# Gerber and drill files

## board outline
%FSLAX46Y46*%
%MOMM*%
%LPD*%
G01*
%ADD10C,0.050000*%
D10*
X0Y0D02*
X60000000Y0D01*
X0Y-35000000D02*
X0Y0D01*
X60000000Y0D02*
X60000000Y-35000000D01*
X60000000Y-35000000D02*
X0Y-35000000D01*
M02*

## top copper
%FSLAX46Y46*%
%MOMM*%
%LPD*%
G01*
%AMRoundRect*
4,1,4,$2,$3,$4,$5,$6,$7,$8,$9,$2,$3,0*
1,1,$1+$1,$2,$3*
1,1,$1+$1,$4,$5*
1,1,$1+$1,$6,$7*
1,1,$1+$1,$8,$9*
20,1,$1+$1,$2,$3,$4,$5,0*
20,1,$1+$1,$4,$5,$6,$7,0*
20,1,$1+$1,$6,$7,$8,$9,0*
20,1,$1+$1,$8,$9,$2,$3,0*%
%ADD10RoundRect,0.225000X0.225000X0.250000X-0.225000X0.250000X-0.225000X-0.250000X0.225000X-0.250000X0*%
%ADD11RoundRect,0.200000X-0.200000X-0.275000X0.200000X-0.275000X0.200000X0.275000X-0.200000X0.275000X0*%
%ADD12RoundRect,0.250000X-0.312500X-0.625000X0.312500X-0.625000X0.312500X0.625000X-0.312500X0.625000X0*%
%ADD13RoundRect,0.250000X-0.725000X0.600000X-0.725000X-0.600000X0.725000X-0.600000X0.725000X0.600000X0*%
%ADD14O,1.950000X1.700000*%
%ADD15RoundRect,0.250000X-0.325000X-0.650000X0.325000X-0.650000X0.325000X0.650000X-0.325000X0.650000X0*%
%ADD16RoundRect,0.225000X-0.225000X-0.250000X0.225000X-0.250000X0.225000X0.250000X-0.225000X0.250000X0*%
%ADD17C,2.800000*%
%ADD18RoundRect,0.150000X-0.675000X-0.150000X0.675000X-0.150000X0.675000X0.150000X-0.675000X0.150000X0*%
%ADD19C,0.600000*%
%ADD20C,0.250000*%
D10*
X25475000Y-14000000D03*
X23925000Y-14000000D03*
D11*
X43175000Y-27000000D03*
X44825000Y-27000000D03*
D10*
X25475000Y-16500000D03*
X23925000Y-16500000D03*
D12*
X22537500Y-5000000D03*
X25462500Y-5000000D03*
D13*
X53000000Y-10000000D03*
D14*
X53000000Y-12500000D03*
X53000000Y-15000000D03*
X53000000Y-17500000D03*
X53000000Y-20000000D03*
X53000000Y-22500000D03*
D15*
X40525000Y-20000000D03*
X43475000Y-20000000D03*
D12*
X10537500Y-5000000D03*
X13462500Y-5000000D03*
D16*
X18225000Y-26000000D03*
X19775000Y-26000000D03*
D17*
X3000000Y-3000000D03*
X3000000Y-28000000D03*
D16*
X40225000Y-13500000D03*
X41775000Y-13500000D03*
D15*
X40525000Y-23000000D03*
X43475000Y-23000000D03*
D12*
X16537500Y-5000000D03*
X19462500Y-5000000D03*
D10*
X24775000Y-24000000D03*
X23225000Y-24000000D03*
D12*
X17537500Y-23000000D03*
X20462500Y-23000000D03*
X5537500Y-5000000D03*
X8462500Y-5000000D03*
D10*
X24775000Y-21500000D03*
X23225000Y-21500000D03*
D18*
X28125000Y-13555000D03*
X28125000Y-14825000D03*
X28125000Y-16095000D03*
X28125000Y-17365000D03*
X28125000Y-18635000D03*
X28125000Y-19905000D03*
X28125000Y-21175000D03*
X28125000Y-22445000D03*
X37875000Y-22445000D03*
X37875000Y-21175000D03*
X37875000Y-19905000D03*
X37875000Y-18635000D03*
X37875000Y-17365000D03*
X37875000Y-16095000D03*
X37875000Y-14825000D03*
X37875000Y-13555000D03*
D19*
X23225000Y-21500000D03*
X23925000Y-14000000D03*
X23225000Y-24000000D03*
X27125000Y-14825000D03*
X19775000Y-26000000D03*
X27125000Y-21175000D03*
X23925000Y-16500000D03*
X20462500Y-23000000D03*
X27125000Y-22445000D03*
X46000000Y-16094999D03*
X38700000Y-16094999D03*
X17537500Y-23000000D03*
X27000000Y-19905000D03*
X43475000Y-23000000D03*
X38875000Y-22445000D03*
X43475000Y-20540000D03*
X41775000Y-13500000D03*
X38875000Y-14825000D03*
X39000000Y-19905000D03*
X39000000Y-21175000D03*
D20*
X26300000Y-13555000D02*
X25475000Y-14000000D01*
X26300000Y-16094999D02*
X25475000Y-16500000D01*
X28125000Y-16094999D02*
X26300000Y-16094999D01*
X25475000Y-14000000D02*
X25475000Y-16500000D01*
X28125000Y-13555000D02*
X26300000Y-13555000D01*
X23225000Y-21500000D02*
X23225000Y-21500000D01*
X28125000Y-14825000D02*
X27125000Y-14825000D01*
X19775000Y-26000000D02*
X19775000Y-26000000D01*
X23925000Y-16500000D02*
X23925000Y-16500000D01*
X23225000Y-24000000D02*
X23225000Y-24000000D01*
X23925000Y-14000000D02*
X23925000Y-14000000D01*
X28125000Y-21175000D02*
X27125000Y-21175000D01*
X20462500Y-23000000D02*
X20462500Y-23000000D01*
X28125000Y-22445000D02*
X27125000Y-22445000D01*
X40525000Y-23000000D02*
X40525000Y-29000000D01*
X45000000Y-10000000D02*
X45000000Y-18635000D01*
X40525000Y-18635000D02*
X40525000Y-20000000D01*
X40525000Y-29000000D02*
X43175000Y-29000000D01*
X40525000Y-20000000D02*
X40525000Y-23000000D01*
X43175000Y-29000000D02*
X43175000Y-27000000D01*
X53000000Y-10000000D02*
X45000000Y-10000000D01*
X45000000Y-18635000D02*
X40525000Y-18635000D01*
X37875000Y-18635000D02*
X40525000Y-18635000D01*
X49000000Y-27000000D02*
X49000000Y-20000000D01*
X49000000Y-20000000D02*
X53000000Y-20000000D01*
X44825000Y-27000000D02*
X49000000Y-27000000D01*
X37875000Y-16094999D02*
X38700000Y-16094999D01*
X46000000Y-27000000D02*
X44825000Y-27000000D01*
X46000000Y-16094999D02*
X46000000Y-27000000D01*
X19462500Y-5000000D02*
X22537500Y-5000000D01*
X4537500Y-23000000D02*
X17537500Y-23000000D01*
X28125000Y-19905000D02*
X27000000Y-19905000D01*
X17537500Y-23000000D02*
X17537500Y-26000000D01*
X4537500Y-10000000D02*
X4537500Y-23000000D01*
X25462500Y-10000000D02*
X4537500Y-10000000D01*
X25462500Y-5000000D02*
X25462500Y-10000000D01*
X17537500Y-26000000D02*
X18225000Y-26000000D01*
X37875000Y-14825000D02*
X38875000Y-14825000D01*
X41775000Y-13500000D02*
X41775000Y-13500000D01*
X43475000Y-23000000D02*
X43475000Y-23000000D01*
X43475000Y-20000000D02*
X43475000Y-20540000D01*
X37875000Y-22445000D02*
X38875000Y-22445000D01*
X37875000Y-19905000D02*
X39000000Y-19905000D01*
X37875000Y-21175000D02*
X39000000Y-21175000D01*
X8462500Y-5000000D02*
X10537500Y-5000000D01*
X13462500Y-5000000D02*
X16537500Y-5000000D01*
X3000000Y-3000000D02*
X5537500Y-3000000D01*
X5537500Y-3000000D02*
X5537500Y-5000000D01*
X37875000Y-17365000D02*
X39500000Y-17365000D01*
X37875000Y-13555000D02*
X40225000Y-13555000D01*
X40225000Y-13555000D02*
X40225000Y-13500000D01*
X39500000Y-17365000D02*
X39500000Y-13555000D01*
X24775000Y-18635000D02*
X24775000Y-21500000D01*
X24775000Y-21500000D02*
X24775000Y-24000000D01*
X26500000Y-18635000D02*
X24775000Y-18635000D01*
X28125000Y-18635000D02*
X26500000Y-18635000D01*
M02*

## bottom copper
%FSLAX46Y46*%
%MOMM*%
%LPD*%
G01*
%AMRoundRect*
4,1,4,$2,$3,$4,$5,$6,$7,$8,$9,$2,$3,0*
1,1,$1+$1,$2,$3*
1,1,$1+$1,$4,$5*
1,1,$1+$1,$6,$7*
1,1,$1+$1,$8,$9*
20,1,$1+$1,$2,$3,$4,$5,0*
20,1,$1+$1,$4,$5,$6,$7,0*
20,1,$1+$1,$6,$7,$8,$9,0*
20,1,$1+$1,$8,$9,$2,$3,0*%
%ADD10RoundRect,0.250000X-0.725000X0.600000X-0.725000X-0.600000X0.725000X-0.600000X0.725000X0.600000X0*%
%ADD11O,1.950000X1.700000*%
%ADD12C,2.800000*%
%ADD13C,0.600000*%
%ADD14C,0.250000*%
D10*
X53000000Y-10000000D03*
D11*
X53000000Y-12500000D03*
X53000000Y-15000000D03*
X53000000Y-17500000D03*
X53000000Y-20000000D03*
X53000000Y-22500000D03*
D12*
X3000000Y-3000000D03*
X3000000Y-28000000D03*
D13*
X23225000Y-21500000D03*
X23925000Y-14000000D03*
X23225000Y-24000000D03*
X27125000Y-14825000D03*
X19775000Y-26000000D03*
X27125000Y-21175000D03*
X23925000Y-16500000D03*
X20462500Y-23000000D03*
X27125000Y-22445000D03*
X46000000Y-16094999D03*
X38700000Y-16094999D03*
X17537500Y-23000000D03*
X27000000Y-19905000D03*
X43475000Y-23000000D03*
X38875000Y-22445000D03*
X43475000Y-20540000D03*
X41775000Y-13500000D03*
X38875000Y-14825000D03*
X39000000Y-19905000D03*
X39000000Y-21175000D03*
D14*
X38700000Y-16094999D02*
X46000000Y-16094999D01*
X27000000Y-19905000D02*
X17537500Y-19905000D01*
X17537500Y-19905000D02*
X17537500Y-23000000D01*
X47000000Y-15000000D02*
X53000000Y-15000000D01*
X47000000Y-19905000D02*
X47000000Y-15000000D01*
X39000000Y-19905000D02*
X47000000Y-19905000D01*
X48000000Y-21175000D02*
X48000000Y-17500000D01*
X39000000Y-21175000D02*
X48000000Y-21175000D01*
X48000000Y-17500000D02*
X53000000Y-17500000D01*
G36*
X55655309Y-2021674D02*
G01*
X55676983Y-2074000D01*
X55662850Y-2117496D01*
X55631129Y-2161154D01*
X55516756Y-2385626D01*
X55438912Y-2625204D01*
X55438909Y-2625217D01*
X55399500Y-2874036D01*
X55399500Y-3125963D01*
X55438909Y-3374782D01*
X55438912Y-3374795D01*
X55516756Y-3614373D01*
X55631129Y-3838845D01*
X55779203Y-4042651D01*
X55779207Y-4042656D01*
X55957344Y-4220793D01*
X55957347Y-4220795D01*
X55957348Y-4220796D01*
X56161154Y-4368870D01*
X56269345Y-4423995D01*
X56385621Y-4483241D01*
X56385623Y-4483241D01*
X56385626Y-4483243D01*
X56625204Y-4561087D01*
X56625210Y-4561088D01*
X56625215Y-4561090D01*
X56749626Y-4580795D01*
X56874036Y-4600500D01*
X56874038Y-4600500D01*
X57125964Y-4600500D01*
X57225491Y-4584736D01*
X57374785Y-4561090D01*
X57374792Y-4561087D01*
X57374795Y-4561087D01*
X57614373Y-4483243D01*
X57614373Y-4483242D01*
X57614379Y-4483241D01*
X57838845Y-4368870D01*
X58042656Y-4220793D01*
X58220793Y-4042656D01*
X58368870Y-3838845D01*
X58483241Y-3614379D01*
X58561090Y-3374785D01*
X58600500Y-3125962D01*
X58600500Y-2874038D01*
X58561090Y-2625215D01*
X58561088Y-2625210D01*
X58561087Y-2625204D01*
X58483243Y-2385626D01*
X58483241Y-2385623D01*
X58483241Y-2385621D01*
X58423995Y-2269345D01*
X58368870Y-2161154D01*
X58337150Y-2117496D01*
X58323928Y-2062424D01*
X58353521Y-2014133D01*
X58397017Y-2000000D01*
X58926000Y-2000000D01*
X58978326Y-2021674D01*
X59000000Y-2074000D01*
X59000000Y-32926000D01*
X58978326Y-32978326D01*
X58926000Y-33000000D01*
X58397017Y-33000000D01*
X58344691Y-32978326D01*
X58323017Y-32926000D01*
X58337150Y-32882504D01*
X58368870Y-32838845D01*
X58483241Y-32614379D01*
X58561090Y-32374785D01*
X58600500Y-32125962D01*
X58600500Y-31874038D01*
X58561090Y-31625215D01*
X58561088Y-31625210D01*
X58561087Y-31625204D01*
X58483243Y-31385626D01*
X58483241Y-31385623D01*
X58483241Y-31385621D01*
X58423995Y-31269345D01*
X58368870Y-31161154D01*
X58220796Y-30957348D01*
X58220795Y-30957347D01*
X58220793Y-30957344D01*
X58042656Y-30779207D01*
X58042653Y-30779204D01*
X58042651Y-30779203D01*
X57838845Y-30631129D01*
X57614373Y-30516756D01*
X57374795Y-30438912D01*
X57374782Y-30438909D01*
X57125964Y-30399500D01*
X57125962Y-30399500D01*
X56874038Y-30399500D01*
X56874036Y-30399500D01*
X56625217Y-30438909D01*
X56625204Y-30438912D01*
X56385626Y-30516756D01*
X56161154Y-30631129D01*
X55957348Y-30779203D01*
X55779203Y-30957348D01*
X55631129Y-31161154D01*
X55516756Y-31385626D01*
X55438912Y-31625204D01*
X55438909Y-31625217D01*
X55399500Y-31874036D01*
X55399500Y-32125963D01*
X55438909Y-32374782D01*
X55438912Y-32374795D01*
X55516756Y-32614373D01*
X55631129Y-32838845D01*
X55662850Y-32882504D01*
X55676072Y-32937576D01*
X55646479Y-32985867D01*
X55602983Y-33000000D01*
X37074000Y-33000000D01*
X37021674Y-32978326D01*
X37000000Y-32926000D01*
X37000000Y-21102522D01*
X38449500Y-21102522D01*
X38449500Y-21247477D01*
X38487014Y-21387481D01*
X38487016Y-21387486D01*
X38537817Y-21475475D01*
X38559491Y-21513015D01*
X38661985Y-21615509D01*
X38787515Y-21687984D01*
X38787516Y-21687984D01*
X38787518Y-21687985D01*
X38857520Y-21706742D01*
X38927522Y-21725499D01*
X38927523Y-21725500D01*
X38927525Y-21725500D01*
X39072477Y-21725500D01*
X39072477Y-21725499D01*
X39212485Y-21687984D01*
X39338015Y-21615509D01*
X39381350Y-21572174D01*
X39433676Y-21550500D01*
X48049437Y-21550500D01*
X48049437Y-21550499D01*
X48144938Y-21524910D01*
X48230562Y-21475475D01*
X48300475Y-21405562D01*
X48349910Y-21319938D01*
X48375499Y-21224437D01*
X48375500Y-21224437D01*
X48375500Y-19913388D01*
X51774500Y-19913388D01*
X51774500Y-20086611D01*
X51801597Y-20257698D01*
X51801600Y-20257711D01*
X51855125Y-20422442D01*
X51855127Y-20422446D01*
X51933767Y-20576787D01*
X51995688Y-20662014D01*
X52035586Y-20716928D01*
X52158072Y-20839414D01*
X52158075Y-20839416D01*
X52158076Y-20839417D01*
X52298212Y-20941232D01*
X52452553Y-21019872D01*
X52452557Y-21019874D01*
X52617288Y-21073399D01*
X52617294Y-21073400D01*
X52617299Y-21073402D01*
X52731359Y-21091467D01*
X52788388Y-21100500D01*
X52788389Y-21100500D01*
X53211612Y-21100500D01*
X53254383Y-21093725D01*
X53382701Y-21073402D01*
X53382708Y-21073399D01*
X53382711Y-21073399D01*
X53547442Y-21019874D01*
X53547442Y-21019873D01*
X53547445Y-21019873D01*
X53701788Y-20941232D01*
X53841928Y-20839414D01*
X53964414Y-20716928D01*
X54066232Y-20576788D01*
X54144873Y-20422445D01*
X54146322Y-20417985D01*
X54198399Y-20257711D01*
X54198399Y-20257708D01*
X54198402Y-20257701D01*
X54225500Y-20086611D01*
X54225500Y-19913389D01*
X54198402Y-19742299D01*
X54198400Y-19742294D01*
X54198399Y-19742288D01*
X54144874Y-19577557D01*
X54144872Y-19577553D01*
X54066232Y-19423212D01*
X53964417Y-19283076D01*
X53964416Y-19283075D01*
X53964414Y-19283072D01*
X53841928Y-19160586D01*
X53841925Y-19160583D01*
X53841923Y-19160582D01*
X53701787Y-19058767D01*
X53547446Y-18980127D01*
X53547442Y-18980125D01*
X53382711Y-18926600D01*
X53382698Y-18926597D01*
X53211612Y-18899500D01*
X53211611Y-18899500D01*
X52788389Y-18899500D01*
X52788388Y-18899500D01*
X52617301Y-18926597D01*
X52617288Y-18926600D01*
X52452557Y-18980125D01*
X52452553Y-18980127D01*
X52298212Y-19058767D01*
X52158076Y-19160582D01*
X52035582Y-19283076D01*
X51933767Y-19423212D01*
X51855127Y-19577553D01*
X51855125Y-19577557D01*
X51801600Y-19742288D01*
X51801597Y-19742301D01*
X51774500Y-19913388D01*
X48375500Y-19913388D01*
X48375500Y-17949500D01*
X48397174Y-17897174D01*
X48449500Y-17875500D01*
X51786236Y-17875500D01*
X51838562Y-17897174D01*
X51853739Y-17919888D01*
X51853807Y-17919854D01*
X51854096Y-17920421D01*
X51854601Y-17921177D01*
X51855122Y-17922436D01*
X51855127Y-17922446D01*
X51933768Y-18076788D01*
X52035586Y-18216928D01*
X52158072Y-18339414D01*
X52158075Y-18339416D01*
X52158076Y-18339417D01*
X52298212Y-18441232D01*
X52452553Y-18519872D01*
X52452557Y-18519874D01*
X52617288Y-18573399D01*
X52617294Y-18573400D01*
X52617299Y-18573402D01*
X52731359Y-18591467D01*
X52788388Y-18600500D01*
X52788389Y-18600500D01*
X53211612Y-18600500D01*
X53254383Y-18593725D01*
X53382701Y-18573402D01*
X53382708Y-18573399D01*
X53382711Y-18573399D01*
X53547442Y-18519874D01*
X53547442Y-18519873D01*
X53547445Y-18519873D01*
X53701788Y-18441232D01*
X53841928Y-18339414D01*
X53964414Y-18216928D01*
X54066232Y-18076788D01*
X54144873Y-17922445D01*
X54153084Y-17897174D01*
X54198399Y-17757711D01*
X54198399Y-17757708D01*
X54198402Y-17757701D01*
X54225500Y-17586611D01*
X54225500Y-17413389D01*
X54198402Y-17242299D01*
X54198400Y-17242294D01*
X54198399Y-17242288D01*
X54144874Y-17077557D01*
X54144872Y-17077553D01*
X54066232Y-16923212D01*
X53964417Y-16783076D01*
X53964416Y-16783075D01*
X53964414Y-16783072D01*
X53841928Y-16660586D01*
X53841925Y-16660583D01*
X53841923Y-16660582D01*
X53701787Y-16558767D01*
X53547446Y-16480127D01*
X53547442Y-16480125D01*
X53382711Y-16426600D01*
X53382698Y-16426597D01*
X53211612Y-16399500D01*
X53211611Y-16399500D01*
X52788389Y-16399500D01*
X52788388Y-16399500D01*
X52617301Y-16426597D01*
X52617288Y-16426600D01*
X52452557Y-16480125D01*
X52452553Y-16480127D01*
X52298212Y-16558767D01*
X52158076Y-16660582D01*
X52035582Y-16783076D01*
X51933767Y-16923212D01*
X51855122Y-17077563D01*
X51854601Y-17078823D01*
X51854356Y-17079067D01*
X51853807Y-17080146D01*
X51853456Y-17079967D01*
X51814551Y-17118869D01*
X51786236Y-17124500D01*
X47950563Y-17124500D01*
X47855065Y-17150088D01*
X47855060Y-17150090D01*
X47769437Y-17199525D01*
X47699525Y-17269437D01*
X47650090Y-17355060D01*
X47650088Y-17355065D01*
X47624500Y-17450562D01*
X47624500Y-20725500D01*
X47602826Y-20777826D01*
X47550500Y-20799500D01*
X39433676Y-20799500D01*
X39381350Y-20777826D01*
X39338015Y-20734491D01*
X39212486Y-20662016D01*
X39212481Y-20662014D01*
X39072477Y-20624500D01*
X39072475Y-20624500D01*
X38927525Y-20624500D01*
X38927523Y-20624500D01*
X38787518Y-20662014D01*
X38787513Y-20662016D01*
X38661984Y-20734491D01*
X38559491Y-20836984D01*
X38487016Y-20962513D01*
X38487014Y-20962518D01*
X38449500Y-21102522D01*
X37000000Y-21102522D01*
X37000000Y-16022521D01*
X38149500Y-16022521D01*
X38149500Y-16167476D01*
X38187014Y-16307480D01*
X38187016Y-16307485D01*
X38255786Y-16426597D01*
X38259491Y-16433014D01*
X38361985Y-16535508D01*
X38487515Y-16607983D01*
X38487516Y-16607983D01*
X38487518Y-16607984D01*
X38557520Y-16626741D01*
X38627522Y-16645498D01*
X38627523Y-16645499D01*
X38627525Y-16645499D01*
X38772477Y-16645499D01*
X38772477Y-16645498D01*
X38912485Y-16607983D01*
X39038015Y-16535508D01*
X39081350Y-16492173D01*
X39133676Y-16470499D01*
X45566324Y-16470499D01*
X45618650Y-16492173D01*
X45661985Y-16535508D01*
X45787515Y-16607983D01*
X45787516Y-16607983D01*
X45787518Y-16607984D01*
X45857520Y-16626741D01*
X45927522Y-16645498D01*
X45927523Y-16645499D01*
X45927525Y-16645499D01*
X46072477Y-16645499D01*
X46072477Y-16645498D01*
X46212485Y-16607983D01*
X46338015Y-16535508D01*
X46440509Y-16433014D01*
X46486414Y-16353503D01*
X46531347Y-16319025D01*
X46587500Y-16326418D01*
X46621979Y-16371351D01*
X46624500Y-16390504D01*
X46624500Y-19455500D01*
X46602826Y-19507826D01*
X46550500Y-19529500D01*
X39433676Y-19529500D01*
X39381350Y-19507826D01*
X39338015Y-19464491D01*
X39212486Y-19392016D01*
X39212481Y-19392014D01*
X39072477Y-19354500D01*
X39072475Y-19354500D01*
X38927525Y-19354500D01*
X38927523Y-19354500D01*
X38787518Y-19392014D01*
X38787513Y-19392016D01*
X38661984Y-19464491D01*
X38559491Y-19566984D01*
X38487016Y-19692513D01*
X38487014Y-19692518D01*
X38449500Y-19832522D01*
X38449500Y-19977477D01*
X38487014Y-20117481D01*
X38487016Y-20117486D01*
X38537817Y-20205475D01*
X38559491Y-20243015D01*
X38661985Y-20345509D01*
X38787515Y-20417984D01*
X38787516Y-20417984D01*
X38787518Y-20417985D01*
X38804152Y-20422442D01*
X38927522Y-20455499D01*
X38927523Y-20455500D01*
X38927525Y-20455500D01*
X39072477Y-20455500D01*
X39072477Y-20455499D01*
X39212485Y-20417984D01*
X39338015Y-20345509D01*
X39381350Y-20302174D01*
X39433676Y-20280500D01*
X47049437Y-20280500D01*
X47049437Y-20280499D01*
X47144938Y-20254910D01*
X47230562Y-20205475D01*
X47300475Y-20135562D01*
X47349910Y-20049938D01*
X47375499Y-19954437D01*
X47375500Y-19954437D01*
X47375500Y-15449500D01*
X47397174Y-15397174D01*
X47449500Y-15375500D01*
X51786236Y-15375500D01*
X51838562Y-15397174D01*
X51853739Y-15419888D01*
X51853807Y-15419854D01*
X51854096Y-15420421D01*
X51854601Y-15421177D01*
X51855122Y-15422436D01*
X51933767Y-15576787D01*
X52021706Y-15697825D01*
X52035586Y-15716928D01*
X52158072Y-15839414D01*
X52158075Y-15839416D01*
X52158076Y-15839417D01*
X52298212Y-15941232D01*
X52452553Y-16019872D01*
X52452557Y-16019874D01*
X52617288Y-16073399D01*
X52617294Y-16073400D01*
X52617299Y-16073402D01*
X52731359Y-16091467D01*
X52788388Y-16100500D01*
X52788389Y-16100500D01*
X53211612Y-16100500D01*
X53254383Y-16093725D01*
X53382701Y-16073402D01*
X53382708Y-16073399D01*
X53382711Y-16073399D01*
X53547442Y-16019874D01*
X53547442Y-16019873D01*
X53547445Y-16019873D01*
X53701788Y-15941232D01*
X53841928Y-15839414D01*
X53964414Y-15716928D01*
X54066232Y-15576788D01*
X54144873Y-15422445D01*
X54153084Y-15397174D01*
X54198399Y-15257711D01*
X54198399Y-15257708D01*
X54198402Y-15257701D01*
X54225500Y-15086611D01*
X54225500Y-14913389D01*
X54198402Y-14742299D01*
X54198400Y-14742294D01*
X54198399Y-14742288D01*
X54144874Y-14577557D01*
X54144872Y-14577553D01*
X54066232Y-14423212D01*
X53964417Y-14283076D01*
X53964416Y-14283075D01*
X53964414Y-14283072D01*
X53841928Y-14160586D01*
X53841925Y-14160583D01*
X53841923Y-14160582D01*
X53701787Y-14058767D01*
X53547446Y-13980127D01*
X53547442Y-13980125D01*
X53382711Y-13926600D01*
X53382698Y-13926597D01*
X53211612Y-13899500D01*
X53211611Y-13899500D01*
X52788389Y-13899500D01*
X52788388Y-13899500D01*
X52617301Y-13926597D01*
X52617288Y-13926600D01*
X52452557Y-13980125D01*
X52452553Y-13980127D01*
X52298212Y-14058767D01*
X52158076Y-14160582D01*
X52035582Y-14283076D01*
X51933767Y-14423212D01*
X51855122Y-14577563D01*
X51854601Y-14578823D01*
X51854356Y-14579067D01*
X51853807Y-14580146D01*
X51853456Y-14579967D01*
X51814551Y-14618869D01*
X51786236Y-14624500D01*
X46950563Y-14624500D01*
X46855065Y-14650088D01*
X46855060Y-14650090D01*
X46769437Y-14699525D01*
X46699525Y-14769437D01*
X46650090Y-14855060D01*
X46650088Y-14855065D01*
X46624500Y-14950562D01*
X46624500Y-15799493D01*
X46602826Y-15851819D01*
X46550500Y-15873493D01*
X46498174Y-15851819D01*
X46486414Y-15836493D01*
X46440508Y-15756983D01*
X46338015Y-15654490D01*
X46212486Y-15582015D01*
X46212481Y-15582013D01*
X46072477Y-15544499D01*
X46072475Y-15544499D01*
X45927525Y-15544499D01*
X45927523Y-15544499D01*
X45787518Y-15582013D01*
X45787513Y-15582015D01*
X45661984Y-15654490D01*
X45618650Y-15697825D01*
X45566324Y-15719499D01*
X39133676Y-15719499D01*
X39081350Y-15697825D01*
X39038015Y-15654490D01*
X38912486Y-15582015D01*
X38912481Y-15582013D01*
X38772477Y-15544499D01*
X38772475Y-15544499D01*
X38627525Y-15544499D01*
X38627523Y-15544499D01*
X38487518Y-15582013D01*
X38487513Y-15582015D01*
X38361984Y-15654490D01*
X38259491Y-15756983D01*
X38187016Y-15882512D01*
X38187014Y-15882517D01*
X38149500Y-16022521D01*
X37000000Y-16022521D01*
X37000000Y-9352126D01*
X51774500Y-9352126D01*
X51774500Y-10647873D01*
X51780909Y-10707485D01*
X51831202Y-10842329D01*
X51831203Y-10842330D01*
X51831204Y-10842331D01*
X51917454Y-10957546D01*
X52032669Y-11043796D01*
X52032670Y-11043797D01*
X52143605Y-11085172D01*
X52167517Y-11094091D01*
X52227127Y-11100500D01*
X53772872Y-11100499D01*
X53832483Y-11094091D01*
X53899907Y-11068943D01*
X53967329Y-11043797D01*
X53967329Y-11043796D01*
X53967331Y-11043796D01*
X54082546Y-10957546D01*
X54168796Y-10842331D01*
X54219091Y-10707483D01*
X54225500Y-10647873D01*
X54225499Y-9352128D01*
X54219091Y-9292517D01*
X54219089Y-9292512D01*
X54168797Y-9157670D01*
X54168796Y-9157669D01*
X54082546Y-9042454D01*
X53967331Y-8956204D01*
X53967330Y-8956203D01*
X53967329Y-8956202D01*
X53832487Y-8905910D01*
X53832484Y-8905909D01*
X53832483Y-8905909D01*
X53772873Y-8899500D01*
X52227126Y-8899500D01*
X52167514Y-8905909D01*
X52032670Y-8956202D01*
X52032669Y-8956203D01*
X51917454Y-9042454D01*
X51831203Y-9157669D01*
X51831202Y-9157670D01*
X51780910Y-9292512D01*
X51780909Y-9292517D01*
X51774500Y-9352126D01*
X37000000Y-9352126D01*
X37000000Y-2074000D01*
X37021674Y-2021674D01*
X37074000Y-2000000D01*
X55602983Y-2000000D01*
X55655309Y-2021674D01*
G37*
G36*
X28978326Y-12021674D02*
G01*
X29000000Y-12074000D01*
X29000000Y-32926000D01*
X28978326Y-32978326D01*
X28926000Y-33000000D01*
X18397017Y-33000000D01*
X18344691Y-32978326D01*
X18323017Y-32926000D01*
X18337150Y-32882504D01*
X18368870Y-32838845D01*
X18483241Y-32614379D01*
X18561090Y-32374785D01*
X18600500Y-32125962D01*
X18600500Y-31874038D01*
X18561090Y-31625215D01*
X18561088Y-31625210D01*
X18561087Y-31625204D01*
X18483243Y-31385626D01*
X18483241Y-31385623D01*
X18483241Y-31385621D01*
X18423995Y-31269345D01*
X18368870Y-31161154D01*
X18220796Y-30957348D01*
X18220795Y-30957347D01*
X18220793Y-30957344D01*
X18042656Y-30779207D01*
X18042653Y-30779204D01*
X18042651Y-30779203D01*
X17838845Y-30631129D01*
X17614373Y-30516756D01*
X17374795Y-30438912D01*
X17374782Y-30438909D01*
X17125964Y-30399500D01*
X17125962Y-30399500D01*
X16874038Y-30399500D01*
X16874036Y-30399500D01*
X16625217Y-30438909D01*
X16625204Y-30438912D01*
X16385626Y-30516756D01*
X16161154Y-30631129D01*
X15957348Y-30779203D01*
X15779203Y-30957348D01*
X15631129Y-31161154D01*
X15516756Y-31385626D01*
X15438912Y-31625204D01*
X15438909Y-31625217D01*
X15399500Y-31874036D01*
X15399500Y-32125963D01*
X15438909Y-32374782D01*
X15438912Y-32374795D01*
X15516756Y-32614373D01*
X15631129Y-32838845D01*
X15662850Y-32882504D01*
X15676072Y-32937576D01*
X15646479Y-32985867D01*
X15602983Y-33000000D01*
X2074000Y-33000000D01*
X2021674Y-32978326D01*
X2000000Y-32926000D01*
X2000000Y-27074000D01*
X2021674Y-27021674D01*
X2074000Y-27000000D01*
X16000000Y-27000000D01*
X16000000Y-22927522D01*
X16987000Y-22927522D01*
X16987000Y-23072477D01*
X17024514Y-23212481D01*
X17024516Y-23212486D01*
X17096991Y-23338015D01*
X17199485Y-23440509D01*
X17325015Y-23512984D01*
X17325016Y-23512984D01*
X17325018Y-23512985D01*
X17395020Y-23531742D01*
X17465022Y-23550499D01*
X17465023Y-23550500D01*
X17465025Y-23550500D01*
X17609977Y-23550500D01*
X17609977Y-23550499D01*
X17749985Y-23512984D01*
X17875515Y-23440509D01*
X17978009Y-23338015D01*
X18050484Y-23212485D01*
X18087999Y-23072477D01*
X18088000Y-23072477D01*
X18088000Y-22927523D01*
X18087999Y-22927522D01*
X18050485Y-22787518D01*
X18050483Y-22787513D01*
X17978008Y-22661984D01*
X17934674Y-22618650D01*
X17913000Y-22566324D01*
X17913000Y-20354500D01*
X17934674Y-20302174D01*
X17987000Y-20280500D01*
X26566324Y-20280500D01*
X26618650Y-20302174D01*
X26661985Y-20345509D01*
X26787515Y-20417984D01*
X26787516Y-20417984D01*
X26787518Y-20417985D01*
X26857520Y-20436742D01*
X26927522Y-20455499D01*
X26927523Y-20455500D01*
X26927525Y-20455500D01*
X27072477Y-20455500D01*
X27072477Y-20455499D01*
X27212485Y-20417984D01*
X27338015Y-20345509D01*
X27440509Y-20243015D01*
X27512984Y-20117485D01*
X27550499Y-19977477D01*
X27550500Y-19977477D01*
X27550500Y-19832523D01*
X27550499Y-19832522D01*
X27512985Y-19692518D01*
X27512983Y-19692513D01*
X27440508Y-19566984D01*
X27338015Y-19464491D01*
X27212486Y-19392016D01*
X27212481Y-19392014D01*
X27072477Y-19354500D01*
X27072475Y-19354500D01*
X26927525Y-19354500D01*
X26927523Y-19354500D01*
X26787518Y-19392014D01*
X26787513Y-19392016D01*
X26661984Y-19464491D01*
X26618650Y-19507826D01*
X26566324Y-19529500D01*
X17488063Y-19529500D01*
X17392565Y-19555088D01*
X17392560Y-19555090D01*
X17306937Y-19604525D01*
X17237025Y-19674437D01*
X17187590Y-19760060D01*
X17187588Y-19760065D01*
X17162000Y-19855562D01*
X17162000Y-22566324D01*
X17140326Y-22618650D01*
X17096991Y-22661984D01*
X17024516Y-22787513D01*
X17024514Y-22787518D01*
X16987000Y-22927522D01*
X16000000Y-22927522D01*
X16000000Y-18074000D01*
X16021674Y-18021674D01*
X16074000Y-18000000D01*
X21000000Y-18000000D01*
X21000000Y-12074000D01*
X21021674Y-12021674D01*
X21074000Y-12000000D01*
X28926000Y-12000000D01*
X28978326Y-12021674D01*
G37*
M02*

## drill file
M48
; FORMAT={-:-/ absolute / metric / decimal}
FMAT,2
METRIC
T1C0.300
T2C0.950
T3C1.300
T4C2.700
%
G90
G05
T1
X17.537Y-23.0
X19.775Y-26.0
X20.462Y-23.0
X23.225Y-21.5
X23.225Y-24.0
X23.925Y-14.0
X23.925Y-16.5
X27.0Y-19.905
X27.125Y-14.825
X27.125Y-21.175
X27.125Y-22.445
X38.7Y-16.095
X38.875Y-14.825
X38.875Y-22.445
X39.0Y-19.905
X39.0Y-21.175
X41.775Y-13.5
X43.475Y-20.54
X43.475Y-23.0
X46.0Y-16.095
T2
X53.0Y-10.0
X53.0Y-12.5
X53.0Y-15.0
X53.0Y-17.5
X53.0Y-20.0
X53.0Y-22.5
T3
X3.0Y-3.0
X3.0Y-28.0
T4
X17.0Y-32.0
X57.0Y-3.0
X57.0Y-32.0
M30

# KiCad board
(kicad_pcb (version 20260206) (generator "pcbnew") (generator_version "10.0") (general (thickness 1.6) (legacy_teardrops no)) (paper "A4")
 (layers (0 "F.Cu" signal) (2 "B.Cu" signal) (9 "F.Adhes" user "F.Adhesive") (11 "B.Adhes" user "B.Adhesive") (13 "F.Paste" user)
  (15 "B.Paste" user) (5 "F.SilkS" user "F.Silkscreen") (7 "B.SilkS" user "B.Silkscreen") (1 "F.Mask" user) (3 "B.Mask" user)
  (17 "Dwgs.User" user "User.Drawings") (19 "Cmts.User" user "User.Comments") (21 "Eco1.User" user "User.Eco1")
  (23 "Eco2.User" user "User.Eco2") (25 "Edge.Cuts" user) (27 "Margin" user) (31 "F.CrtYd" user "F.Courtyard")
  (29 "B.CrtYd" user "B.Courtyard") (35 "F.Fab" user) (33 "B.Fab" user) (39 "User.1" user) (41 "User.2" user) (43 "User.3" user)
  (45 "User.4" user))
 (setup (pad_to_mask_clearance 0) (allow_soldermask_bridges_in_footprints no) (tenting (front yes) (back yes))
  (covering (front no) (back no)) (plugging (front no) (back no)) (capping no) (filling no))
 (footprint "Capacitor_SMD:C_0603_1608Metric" (layer "F.Cu") (at 24.7 14 180)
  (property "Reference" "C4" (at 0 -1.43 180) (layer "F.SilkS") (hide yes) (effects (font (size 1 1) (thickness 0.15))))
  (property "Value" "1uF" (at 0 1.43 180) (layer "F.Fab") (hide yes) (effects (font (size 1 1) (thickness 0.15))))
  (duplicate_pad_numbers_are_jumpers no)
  (pad "1" smd roundrect (at -0.775 0 180) (size 0.9 0.95) (layers "F.Cu" "F.Mask" "F.Paste") (roundrect_rratio 0.25) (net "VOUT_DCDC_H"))
  (pad "2" smd roundrect (at 0.775 0 180) (size 0.9 0.95) (layers "F.Cu" "F.Mask" "F.Paste") (roundrect_rratio 0.25) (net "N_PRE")))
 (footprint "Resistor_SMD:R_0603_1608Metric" (layer "F.Cu") (at 44 27)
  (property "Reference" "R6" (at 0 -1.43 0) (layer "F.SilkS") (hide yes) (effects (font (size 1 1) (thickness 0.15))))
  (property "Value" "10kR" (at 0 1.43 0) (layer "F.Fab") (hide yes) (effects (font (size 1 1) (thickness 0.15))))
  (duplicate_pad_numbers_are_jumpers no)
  (pad "1" smd roundrect (at -0.825 0) (size 0.8 0.95) (layers "F.Cu" "F.Mask" "F.Paste") (roundrect_rratio 0.25) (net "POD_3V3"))
  (pad "2" smd roundrect (at 0.825 0) (size 0.8 0.95) (layers "F.Cu" "F.Mask" "F.Paste") (roundrect_rratio 0.25) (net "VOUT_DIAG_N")))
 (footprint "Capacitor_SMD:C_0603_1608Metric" (layer "F.Cu") (at 24.7 16.5 180)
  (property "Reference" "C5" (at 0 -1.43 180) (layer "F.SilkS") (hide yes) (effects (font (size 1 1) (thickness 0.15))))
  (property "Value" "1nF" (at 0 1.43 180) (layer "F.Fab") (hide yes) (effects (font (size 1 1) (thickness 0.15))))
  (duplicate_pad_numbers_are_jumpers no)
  (pad "1" smd roundrect (at -0.775 0 180) (size 0.9 0.95) (layers "F.Cu" "F.Mask" "F.Paste") (roundrect_rratio 0.25) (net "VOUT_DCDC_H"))
  (pad "2" smd roundrect (at 0.775 0 180) (size 0.9 0.95) (layers "F.Cu" "F.Mask" "F.Paste") (roundrect_rratio 0.25) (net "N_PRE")))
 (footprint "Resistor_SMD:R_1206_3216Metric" (layer "F.Cu") (at 24 5)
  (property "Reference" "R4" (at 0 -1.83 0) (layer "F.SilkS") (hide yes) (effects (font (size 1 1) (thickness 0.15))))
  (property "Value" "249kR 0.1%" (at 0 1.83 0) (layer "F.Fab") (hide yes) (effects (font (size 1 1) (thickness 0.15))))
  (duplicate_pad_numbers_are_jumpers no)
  (pad "1" smd roundrect (at -1.4625 0) (size 1.125 1.75) (layers "F.Cu" "F.Mask" "F.Paste") (roundrect_rratio 0.222222) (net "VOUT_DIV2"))
  (pad "2" smd roundrect (at 1.4625 0) (size 1.125 1.75) (layers "F.Cu" "F.Mask" "F.Paste") (roundrect_rratio 0.222222) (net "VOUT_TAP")))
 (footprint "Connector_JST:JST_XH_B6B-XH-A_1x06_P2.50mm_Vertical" (layer "F.Cu") (at 53 10 -90)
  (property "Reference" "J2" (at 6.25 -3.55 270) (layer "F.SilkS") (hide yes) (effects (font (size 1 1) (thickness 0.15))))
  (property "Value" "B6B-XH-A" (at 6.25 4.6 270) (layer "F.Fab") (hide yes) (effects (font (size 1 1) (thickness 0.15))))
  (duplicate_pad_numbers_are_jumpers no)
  (pad "1" thru_hole roundrect (at 0 0 270) (size 1.7 1.95) (drill 0.95) (layers "*.Cu" "*.Mask") (remove_unused_layers no)
   (roundrect_rratio 0.147059) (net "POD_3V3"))
  (pad "2" thru_hole oval (at 2.5 0 270) (size 1.7 1.95) (drill 0.95) (layers "*.Cu" "*.Mask") (remove_unused_layers no) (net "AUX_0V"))
  (pad "3" thru_hole oval (at 5 0 270) (size 1.7 1.95) (drill 0.95) (layers "*.Cu" "*.Mask") (remove_unused_layers no) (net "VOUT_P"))
  (pad "4" thru_hole oval (at 7.5 0 270) (size 1.7 1.95) (drill 0.95) (layers "*.Cu" "*.Mask") (remove_unused_layers no) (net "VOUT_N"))
  (pad "5" thru_hole oval (at 10 0 270) (size 1.7 1.95) (drill 0.95) (layers "*.Cu" "*.Mask") (remove_unused_layers no) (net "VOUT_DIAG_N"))
  (pad "6" thru_hole oval (at 12.5 0 270) (size 1.7 1.95) (drill 0.95) (layers "*.Cu" "*.Mask") (remove_unused_layers no) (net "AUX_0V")))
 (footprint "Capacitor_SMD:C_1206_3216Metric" (layer "F.Cu") (at 42 20)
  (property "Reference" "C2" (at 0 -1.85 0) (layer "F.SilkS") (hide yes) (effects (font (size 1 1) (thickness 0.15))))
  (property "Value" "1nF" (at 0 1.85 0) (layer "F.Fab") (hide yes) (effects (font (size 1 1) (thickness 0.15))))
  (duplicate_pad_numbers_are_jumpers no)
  (pad "1" smd roundrect (at -1.475 0) (size 1.15 1.8) (layers "F.Cu" "F.Mask" "F.Paste") (roundrect_rratio 0.217391) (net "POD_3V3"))
  (pad "2" smd roundrect (at 1.475 0) (size 1.15 1.8) (layers "F.Cu" "F.Mask" "F.Paste") (roundrect_rratio 0.217391) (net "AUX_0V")))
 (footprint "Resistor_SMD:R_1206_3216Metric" (layer "F.Cu") (at 12 5)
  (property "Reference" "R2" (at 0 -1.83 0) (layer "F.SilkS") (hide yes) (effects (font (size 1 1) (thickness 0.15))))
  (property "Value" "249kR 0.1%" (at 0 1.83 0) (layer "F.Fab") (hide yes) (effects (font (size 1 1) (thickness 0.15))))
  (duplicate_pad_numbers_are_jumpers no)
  (pad "1" smd roundrect (at -1.4625 0) (size 1.125 1.75) (layers "F.Cu" "F.Mask" "F.Paste") (roundrect_rratio 0.222222) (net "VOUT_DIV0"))
  (pad "2" smd roundrect (at 1.4625 0) (size 1.125 1.75) (layers "F.Cu" "F.Mask" "F.Paste") (roundrect_rratio 0.222222) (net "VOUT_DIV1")))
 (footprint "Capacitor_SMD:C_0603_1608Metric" (layer "F.Cu") (at 19 26)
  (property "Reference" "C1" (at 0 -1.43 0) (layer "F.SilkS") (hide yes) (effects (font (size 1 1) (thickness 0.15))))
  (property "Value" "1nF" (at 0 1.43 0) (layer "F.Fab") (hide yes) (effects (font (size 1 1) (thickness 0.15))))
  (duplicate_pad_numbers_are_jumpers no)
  (pad "1" smd roundrect (at -0.775 0) (size 0.9 0.95) (layers "F.Cu" "F.Mask" "F.Paste") (roundrect_rratio 0.25) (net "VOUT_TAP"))
  (pad "2" smd roundrect (at 0.775 0) (size 0.9 0.95) (layers "F.Cu" "F.Mask" "F.Paste") (roundrect_rratio 0.25) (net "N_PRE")))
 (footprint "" (layer "F.Cu") (at 57 32)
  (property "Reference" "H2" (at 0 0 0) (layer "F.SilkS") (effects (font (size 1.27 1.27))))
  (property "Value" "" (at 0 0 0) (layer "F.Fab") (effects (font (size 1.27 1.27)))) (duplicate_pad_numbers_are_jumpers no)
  (pad "" np_thru_hole circle (at 0 0) (size 2.7 2.7) (drill 2.7) (layers "*.Cu")))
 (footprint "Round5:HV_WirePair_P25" (layer "F.Cu") (at 3 3)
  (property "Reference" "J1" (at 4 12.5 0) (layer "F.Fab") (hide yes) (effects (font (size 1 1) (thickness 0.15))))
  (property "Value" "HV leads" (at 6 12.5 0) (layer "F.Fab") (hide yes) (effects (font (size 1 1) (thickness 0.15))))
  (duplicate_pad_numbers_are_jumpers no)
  (pad "1" thru_hole circle (at 0 0) (size 2.8 2.8) (drill 1.3) (layers "*.Cu" "*.Mask") (remove_unused_layers no) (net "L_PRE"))
  (pad "2" thru_hole circle (at 0 25) (size 2.8 2.8) (drill 1.3) (layers "*.Cu" "*.Mask") (remove_unused_layers no) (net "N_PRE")))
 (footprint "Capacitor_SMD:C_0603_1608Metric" (layer "F.Cu") (at 41 13.5)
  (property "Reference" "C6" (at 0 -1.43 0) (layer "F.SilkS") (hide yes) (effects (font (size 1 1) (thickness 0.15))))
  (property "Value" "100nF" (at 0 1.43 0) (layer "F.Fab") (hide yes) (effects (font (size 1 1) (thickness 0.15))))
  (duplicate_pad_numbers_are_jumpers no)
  (pad "1" smd roundrect (at -0.775 0) (size 0.9 0.95) (layers "F.Cu" "F.Mask" "F.Paste") (roundrect_rratio 0.25) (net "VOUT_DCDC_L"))
  (pad "2" smd roundrect (at 0.775 0) (size 0.9 0.95) (layers "F.Cu" "F.Mask" "F.Paste") (roundrect_rratio 0.25) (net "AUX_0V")))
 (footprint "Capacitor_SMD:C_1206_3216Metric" (layer "F.Cu") (at 42 23)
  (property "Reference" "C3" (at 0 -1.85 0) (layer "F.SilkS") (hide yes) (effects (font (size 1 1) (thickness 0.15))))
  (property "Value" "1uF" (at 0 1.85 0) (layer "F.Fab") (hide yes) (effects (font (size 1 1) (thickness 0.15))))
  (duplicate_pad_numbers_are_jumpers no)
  (pad "1" smd roundrect (at -1.475 0) (size 1.15 1.8) (layers "F.Cu" "F.Mask" "F.Paste") (roundrect_rratio 0.217391) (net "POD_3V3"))
  (pad "2" smd roundrect (at 1.475 0) (size 1.15 1.8) (layers "F.Cu" "F.Mask" "F.Paste") (roundrect_rratio 0.217391) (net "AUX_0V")))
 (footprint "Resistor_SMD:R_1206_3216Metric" (layer "F.Cu") (at 18 5)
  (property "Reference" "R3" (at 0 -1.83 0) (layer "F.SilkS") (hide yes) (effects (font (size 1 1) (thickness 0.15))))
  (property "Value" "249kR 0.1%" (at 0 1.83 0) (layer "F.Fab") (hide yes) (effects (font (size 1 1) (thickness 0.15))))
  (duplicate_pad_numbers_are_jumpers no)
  (pad "1" smd roundrect (at -1.4625 0) (size 1.125 1.75) (layers "F.Cu" "F.Mask" "F.Paste") (roundrect_rratio 0.222222) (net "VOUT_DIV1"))
  (pad "2" smd roundrect (at 1.4625 0) (size 1.125 1.75) (layers "F.Cu" "F.Mask" "F.Paste") (roundrect_rratio 0.222222) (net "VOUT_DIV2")))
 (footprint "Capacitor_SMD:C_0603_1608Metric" (layer "F.Cu") (at 24 24 180)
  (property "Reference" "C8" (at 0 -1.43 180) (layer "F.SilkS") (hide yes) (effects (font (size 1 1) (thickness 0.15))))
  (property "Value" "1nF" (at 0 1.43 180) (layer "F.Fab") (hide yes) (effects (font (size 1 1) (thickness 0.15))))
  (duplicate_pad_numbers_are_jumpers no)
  (pad "1" smd roundrect (at -0.775 0 180) (size 0.9 0.95) (layers "F.Cu" "F.Mask" "F.Paste") (roundrect_rratio 0.25) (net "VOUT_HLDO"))
  (pad "2" smd roundrect (at 0.775 0 180) (size 0.9 0.95) (layers "F.Cu" "F.Mask" "F.Paste") (roundrect_rratio 0.25) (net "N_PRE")))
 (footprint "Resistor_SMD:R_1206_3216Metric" (layer "F.Cu") (at 19 23)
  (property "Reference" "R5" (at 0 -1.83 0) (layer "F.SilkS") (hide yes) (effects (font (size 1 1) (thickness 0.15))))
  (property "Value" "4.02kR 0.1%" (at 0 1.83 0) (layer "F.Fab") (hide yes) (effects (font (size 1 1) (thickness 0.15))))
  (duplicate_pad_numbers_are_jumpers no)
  (pad "1" smd roundrect (at -1.4625 0) (size 1.125 1.75) (layers "F.Cu" "F.Mask" "F.Paste") (roundrect_rratio 0.222222) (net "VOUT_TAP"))
  (pad "2" smd roundrect (at 1.4625 0) (size 1.125 1.75) (layers "F.Cu" "F.Mask" "F.Paste") (roundrect_rratio 0.222222) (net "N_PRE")))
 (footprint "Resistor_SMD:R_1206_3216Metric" (layer "F.Cu") (at 7 5)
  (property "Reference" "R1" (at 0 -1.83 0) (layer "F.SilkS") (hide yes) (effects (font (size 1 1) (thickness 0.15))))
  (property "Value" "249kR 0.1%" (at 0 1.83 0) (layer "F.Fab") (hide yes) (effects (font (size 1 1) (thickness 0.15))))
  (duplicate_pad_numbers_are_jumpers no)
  (pad "1" smd roundrect (at -1.4625 0) (size 1.125 1.75) (layers "F.Cu" "F.Mask" "F.Paste") (roundrect_rratio 0.222222) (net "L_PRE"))
  (pad "2" smd roundrect (at 1.4625 0) (size 1.125 1.75) (layers "F.Cu" "F.Mask" "F.Paste") (roundrect_rratio 0.222222) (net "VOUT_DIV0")))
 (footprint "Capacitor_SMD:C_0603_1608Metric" (layer "F.Cu") (at 24 21.5 180)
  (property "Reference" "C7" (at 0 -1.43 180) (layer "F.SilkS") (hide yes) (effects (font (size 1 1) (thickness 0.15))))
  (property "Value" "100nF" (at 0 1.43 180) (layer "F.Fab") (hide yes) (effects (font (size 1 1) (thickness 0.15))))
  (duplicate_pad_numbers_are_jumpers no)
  (pad "1" smd roundrect (at -0.775 0 180) (size 0.9 0.95) (layers "F.Cu" "F.Mask" "F.Paste") (roundrect_rratio 0.25) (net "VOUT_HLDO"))
  (pad "2" smd roundrect (at 0.775 0 180) (size 0.9 0.95) (layers "F.Cu" "F.Mask" "F.Paste") (roundrect_rratio 0.25) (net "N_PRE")))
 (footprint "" (layer "F.Cu") (at 57 3)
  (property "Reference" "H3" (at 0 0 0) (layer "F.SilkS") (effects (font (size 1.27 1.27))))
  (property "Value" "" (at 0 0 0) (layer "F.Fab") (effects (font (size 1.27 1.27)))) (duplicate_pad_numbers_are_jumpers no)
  (pad "" np_thru_hole circle (at 0 0) (size 2.7 2.7) (drill 2.7) (layers "*.Cu")))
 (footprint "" (layer "F.Cu") (at 17 32)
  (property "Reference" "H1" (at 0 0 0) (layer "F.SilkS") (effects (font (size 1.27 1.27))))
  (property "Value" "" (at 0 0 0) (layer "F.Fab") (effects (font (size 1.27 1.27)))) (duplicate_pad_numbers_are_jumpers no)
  (pad "" np_thru_hole circle (at 0 0) (size 2.7 2.7) (drill 2.7) (layers "*.Cu")))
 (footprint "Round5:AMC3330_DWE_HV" (layer "F.Cu") (at 33 18)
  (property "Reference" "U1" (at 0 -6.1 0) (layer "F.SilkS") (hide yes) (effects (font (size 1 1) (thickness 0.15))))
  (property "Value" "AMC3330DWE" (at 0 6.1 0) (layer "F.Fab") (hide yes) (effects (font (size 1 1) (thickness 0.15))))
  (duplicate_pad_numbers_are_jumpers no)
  (pad "1" smd roundrect (at -4.875 -4.445) (size 1.65 0.6) (layers "F.Cu" "F.Mask" "F.Paste") (roundrect_rratio 0.25) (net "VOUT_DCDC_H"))
  (pad "2" smd roundrect (at -4.875 -3.175) (size 1.65 0.6) (layers "F.Cu" "F.Mask" "F.Paste") (roundrect_rratio 0.25) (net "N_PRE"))
  (pad "3" smd roundrect (at -4.875 -1.905) (size 1.65 0.6) (layers "F.Cu" "F.Mask" "F.Paste") (roundrect_rratio 0.25) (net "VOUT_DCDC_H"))
  (pad "4" smd roundrect (at -4.875 -0.635) (size 1.65 0.6) (layers "F.Cu" "F.Mask" "F.Paste") (roundrect_rratio 0.25)
   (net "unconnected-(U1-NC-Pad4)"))
  (pad "5" smd roundrect (at -4.875 0.635) (size 1.65 0.6) (layers "F.Cu" "F.Mask" "F.Paste") (roundrect_rratio 0.25) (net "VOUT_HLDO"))
  (pad "6" smd roundrect (at -4.875 1.905) (size 1.65 0.6) (layers "F.Cu" "F.Mask" "F.Paste") (roundrect_rratio 0.25) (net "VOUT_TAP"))
  (pad "7" smd roundrect (at -4.875 3.175) (size 1.65 0.6) (layers "F.Cu" "F.Mask" "F.Paste") (roundrect_rratio 0.25) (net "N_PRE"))
  (pad "8" smd roundrect (at -4.875 4.445) (size 1.65 0.6) (layers "F.Cu" "F.Mask" "F.Paste") (roundrect_rratio 0.25) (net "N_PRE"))
  (pad "9" smd roundrect (at 4.875 4.445) (size 1.65 0.6) (layers "F.Cu" "F.Mask" "F.Paste") (roundrect_rratio 0.25) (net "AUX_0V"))
  (pad "10" smd roundrect (at 4.875 3.175) (size 1.65 0.6) (layers "F.Cu" "F.Mask" "F.Paste") (roundrect_rratio 0.25) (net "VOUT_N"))
  (pad "11" smd roundrect (at 4.875 1.905) (size 1.65 0.6) (layers "F.Cu" "F.Mask" "F.Paste") (roundrect_rratio 0.25) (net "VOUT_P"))
  (pad "12" smd roundrect (at 4.875 0.635) (size 1.65 0.6) (layers "F.Cu" "F.Mask" "F.Paste") (roundrect_rratio 0.25) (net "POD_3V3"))
  (pad "13" smd roundrect (at 4.875 -0.635) (size 1.65 0.6) (layers "F.Cu" "F.Mask" "F.Paste") (roundrect_rratio 0.25) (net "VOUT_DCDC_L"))
  (pad "14" smd roundrect (at 4.875 -1.905) (size 1.65 0.6) (layers "F.Cu" "F.Mask" "F.Paste") (roundrect_rratio 0.25) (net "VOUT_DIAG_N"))
  (pad "15" smd roundrect (at 4.875 -3.175) (size 1.65 0.6) (layers "F.Cu" "F.Mask" "F.Paste") (roundrect_rratio 0.25) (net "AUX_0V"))
  (pad "16" smd roundrect (at 4.875 -4.445) (size 1.65 0.6) (layers "F.Cu" "F.Mask" "F.Paste") (roundrect_rratio 0.25) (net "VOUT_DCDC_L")))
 (gr_line (start 0 0) (end 60 0) (stroke (width 0.05) (type default)) (layer "Edge.Cuts"))
 (gr_line (start 0 35) (end 0 0) (stroke (width 0.05) (type default)) (layer "Edge.Cuts"))
 (gr_line (start 60 0) (end 60 35) (stroke (width 0.05) (type default)) (layer "Edge.Cuts"))
 (gr_line (start 60 35) (end 0 35) (stroke (width 0.05) (type default)) (layer "Edge.Cuts"))
 (segment (start 26.3 13.555) (end 25.475 14) (width 0.25) (layer "F.Cu") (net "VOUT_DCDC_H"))
 (segment (start 26.3 16.094999) (end 25.475 16.5) (width 0.25) (layer "F.Cu") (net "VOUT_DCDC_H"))
 (segment (start 28.125 16.094999) (end 26.3 16.094999) (width 0.25) (layer "F.Cu") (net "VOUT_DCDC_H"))
 (segment (start 25.475 14) (end 25.475 16.5) (width 0.25) (layer "F.Cu") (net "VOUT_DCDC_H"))
 (segment (start 28.125 13.555) (end 26.3 13.555) (width 0.25) (layer "F.Cu") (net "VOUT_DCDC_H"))
 (segment (start 23.225 21.5) (end 23.225 21.5) (width 0.25) (layer "F.Cu") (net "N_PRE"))
 (segment (start 28.125 14.825) (end 27.125 14.825) (width 0.25) (layer "F.Cu") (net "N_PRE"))
 (segment (start 19.775 26) (end 19.775 26) (width 0.25) (layer "F.Cu") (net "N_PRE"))
 (segment (start 23.925 16.5) (end 23.925 16.5) (width 0.25) (layer "F.Cu") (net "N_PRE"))
 (segment (start 23.225 24) (end 23.225 24) (width 0.25) (layer "F.Cu") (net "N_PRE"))
 (segment (start 23.925 14) (end 23.925 14) (width 0.25) (layer "F.Cu") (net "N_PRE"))
 (segment (start 28.125 21.175) (end 27.125 21.175) (width 0.25) (layer "F.Cu") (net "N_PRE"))
 (segment (start 20.4625 23) (end 20.4625 23) (width 0.25) (layer "F.Cu") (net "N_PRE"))
 (segment (start 28.125 22.445) (end 27.125 22.445) (width 0.25) (layer "F.Cu") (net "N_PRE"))
 (via (at 23.225 21.5) (size 0.6) (drill 0.3) (layers "F.Cu" "B.Cu") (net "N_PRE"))
 (via (at 23.925 14) (size 0.6) (drill 0.3) (layers "F.Cu" "B.Cu") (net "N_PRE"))
 (via (at 23.225 24) (size 0.6) (drill 0.3) (layers "F.Cu" "B.Cu") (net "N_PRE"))
 (via (at 27.125 14.825) (size 0.6) (drill 0.3) (layers "F.Cu" "B.Cu") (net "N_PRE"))
 (via (at 19.775 26) (size 0.6) (drill 0.3) (layers "F.Cu" "B.Cu") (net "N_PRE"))
 (via (at 27.125 21.175) (size 0.6) (drill 0.3) (layers "F.Cu" "B.Cu") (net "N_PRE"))
 (via (at 23.925 16.5) (size 0.6) (drill 0.3) (layers "F.Cu" "B.Cu") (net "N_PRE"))
 (via (at 20.4625 23) (size 0.6) (drill 0.3) (layers "F.Cu" "B.Cu") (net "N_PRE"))
 (via (at 27.125 22.445) (size 0.6) (drill 0.3) (layers "F.Cu" "B.Cu") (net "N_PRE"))
 (segment (start 40.525 23) (end 40.525 29) (width 0.25) (layer "F.Cu") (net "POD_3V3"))
 (segment (start 45 10) (end 45 18.635) (width 0.25) (layer "F.Cu") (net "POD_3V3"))
 (segment (start 40.525 18.635) (end 40.525 20) (width 0.25) (layer "F.Cu") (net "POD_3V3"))
 (segment (start 40.525 29) (end 43.175 29) (width 0.25) (layer "F.Cu") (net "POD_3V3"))
 (segment (start 40.525 20) (end 40.525 23) (width 0.25) (layer "F.Cu") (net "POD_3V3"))
 (segment (start 43.175 29) (end 43.175 27) (width 0.25) (layer "F.Cu") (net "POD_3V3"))
 (segment (start 53 10) (end 45 10) (width 0.25) (layer "F.Cu") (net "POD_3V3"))
 (segment (start 45 18.635) (end 40.525 18.635) (width 0.25) (layer "F.Cu") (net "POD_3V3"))
 (segment (start 37.875 18.635) (end 40.525 18.635) (width 0.25) (layer "F.Cu") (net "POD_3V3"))
 (segment (start 49 27) (end 49 20) (width 0.25) (layer "F.Cu") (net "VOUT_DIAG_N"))
 (segment (start 49 20) (end 53 20) (width 0.25) (layer "F.Cu") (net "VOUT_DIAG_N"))
 (segment (start 44.825 27) (end 49 27) (width 0.25) (layer "F.Cu") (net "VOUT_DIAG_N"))
 (segment (start 37.875 16.094999) (end 38.7 16.094999) (width 0.25) (layer "F.Cu") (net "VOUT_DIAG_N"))
 (segment (start 46 27) (end 44.825 27) (width 0.25) (layer "F.Cu") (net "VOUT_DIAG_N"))
 (segment (start 46 16.094999) (end 46 27) (width 0.25) (layer "F.Cu") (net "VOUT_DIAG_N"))
 (via (at 46 16.094999) (size 0.6) (drill 0.3) (layers "F.Cu" "B.Cu") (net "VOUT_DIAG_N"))
 (via (at 38.7 16.094999) (size 0.6) (drill 0.3) (layers "F.Cu" "B.Cu") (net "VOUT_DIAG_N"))
 (segment (start 38.7 16.094999) (end 46 16.094999) (width 0.25) (layer "B.Cu") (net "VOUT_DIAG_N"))
 (segment (start 19.4625 5) (end 22.5375 5) (width 0.25) (layer "F.Cu") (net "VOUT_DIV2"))
 (segment (start 4.5375 23) (end 17.5375 23) (width 0.25) (layer "F.Cu") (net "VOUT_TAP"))
 (segment (start 28.125 19.905) (end 27 19.905) (width 0.25) (layer "F.Cu") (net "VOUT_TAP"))
 (segment (start 17.5375 23) (end 17.5375 26) (width 0.25) (layer "F.Cu") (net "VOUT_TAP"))
 (segment (start 4.5375 10) (end 4.5375 23) (width 0.25) (layer "F.Cu") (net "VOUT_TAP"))
 (segment (start 25.4625 10) (end 4.5375 10) (width 0.25) (layer "F.Cu") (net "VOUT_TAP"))
 (segment (start 25.4625 5) (end 25.4625 10) (width 0.25) (layer "F.Cu") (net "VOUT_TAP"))
 (segment (start 17.5375 26) (end 18.225 26) (width 0.25) (layer "F.Cu") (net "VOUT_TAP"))
 (via (at 17.5375 23) (size 0.6) (drill 0.3) (layers "F.Cu" "B.Cu") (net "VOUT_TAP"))
 (via (at 27 19.905) (size 0.6) (drill 0.3) (layers "F.Cu" "B.Cu") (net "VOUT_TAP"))
 (segment (start 27 19.905) (end 17.5375 19.905) (width 0.25) (layer "B.Cu") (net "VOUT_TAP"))
 (segment (start 17.5375 19.905) (end 17.5375 23) (width 0.25) (layer "B.Cu") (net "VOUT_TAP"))
 (segment (start 37.875 14.825) (end 38.875 14.825) (width 0.25) (layer "F.Cu") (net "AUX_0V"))
 (segment (start 41.775 13.5) (end 41.775 13.5) (width 0.25) (layer "F.Cu") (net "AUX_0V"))
 (segment (start 43.475 23) (end 43.475 23) (width 0.25) (layer "F.Cu") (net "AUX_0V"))
 (segment (start 43.475 20) (end 43.475 20.54) (width 0.25) (layer "F.Cu") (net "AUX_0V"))
 (segment (start 37.875 22.445) (end 38.875 22.445) (width 0.25) (layer "F.Cu") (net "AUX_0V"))
 (via (at 43.475 23) (size 0.6) (drill 0.3) (layers "F.Cu" "B.Cu") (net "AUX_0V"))
 (via (at 38.875 22.445) (size 0.6) (drill 0.3) (layers "F.Cu" "B.Cu") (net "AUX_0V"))
 (via (at 43.475 20.54) (size 0.6) (drill 0.3) (layers "F.Cu" "B.Cu") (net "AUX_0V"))
 (via (at 41.775 13.5) (size 0.6) (drill 0.3) (layers "F.Cu" "B.Cu") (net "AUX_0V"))
 (via (at 38.875 14.825) (size 0.6) (drill 0.3) (layers "F.Cu" "B.Cu") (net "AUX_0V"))
 (segment (start 37.875 19.905) (end 39 19.905) (width 0.25) (layer "F.Cu") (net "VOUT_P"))
 (via (at 39 19.905) (size 0.6) (drill 0.3) (layers "F.Cu" "B.Cu") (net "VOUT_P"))
 (segment (start 47 15) (end 53 15) (width 0.25) (layer "B.Cu") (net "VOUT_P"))
 (segment (start 47 19.905) (end 47 15) (width 0.25) (layer "B.Cu") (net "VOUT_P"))
 (segment (start 39 19.905) (end 47 19.905) (width 0.25) (layer "B.Cu") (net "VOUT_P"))
 (segment (start 37.875 21.175) (end 39 21.175) (width 0.25) (layer "F.Cu") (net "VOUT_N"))
 (via (at 39 21.175) (size 0.6) (drill 0.3) (layers "F.Cu" "B.Cu") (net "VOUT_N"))
 (segment (start 48 21.175) (end 48 17.5) (width 0.25) (layer "B.Cu") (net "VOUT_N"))
 (segment (start 39 21.175) (end 48 21.175) (width 0.25) (layer "B.Cu") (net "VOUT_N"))
 (segment (start 48 17.5) (end 53 17.5) (width 0.25) (layer "B.Cu") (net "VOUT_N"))
 (segment (start 8.4625 5) (end 10.5375 5) (width 0.25) (layer "F.Cu") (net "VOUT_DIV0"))
 (segment (start 13.4625 5) (end 16.5375 5) (width 0.25) (layer "F.Cu") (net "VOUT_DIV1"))
 (segment (start 3 3) (end 5.5375 3) (width 0.25) (layer "F.Cu") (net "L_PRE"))
 (segment (start 5.5375 3) (end 5.5375 5) (width 0.25) (layer "F.Cu") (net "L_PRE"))
 (segment (start 37.875 17.365) (end 39.5 17.365) (width 0.25) (layer "F.Cu") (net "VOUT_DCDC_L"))
 (segment (start 37.875 13.555) (end 40.225 13.555) (width 0.25) (layer "F.Cu") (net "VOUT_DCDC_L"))
 (segment (start 40.225 13.555) (end 40.225 13.5) (width 0.25) (layer "F.Cu") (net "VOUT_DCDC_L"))
 (segment (start 39.5 17.365) (end 39.5 13.555) (width 0.25) (layer "F.Cu") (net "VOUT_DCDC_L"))
 (segment (start 24.775 18.635) (end 24.775 21.5) (width 0.25) (layer "F.Cu") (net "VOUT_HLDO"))
 (segment (start 24.775 21.5) (end 24.775 24) (width 0.25) (layer "F.Cu") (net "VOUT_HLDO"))
 (segment (start 26.5 18.635) (end 24.775 18.635) (width 0.25) (layer "F.Cu") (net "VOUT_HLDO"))
 (segment (start 28.125 18.635) (end 26.5 18.635) (width 0.25) (layer "F.Cu") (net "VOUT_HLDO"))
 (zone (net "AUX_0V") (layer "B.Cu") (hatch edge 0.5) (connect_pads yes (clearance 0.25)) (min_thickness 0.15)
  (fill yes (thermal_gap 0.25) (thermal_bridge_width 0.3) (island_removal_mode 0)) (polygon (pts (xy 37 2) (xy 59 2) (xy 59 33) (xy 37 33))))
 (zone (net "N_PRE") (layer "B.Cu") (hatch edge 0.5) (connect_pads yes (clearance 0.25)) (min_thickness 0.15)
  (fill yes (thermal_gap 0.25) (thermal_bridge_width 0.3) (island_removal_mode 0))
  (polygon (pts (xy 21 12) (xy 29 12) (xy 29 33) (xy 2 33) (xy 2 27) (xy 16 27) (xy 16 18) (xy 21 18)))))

